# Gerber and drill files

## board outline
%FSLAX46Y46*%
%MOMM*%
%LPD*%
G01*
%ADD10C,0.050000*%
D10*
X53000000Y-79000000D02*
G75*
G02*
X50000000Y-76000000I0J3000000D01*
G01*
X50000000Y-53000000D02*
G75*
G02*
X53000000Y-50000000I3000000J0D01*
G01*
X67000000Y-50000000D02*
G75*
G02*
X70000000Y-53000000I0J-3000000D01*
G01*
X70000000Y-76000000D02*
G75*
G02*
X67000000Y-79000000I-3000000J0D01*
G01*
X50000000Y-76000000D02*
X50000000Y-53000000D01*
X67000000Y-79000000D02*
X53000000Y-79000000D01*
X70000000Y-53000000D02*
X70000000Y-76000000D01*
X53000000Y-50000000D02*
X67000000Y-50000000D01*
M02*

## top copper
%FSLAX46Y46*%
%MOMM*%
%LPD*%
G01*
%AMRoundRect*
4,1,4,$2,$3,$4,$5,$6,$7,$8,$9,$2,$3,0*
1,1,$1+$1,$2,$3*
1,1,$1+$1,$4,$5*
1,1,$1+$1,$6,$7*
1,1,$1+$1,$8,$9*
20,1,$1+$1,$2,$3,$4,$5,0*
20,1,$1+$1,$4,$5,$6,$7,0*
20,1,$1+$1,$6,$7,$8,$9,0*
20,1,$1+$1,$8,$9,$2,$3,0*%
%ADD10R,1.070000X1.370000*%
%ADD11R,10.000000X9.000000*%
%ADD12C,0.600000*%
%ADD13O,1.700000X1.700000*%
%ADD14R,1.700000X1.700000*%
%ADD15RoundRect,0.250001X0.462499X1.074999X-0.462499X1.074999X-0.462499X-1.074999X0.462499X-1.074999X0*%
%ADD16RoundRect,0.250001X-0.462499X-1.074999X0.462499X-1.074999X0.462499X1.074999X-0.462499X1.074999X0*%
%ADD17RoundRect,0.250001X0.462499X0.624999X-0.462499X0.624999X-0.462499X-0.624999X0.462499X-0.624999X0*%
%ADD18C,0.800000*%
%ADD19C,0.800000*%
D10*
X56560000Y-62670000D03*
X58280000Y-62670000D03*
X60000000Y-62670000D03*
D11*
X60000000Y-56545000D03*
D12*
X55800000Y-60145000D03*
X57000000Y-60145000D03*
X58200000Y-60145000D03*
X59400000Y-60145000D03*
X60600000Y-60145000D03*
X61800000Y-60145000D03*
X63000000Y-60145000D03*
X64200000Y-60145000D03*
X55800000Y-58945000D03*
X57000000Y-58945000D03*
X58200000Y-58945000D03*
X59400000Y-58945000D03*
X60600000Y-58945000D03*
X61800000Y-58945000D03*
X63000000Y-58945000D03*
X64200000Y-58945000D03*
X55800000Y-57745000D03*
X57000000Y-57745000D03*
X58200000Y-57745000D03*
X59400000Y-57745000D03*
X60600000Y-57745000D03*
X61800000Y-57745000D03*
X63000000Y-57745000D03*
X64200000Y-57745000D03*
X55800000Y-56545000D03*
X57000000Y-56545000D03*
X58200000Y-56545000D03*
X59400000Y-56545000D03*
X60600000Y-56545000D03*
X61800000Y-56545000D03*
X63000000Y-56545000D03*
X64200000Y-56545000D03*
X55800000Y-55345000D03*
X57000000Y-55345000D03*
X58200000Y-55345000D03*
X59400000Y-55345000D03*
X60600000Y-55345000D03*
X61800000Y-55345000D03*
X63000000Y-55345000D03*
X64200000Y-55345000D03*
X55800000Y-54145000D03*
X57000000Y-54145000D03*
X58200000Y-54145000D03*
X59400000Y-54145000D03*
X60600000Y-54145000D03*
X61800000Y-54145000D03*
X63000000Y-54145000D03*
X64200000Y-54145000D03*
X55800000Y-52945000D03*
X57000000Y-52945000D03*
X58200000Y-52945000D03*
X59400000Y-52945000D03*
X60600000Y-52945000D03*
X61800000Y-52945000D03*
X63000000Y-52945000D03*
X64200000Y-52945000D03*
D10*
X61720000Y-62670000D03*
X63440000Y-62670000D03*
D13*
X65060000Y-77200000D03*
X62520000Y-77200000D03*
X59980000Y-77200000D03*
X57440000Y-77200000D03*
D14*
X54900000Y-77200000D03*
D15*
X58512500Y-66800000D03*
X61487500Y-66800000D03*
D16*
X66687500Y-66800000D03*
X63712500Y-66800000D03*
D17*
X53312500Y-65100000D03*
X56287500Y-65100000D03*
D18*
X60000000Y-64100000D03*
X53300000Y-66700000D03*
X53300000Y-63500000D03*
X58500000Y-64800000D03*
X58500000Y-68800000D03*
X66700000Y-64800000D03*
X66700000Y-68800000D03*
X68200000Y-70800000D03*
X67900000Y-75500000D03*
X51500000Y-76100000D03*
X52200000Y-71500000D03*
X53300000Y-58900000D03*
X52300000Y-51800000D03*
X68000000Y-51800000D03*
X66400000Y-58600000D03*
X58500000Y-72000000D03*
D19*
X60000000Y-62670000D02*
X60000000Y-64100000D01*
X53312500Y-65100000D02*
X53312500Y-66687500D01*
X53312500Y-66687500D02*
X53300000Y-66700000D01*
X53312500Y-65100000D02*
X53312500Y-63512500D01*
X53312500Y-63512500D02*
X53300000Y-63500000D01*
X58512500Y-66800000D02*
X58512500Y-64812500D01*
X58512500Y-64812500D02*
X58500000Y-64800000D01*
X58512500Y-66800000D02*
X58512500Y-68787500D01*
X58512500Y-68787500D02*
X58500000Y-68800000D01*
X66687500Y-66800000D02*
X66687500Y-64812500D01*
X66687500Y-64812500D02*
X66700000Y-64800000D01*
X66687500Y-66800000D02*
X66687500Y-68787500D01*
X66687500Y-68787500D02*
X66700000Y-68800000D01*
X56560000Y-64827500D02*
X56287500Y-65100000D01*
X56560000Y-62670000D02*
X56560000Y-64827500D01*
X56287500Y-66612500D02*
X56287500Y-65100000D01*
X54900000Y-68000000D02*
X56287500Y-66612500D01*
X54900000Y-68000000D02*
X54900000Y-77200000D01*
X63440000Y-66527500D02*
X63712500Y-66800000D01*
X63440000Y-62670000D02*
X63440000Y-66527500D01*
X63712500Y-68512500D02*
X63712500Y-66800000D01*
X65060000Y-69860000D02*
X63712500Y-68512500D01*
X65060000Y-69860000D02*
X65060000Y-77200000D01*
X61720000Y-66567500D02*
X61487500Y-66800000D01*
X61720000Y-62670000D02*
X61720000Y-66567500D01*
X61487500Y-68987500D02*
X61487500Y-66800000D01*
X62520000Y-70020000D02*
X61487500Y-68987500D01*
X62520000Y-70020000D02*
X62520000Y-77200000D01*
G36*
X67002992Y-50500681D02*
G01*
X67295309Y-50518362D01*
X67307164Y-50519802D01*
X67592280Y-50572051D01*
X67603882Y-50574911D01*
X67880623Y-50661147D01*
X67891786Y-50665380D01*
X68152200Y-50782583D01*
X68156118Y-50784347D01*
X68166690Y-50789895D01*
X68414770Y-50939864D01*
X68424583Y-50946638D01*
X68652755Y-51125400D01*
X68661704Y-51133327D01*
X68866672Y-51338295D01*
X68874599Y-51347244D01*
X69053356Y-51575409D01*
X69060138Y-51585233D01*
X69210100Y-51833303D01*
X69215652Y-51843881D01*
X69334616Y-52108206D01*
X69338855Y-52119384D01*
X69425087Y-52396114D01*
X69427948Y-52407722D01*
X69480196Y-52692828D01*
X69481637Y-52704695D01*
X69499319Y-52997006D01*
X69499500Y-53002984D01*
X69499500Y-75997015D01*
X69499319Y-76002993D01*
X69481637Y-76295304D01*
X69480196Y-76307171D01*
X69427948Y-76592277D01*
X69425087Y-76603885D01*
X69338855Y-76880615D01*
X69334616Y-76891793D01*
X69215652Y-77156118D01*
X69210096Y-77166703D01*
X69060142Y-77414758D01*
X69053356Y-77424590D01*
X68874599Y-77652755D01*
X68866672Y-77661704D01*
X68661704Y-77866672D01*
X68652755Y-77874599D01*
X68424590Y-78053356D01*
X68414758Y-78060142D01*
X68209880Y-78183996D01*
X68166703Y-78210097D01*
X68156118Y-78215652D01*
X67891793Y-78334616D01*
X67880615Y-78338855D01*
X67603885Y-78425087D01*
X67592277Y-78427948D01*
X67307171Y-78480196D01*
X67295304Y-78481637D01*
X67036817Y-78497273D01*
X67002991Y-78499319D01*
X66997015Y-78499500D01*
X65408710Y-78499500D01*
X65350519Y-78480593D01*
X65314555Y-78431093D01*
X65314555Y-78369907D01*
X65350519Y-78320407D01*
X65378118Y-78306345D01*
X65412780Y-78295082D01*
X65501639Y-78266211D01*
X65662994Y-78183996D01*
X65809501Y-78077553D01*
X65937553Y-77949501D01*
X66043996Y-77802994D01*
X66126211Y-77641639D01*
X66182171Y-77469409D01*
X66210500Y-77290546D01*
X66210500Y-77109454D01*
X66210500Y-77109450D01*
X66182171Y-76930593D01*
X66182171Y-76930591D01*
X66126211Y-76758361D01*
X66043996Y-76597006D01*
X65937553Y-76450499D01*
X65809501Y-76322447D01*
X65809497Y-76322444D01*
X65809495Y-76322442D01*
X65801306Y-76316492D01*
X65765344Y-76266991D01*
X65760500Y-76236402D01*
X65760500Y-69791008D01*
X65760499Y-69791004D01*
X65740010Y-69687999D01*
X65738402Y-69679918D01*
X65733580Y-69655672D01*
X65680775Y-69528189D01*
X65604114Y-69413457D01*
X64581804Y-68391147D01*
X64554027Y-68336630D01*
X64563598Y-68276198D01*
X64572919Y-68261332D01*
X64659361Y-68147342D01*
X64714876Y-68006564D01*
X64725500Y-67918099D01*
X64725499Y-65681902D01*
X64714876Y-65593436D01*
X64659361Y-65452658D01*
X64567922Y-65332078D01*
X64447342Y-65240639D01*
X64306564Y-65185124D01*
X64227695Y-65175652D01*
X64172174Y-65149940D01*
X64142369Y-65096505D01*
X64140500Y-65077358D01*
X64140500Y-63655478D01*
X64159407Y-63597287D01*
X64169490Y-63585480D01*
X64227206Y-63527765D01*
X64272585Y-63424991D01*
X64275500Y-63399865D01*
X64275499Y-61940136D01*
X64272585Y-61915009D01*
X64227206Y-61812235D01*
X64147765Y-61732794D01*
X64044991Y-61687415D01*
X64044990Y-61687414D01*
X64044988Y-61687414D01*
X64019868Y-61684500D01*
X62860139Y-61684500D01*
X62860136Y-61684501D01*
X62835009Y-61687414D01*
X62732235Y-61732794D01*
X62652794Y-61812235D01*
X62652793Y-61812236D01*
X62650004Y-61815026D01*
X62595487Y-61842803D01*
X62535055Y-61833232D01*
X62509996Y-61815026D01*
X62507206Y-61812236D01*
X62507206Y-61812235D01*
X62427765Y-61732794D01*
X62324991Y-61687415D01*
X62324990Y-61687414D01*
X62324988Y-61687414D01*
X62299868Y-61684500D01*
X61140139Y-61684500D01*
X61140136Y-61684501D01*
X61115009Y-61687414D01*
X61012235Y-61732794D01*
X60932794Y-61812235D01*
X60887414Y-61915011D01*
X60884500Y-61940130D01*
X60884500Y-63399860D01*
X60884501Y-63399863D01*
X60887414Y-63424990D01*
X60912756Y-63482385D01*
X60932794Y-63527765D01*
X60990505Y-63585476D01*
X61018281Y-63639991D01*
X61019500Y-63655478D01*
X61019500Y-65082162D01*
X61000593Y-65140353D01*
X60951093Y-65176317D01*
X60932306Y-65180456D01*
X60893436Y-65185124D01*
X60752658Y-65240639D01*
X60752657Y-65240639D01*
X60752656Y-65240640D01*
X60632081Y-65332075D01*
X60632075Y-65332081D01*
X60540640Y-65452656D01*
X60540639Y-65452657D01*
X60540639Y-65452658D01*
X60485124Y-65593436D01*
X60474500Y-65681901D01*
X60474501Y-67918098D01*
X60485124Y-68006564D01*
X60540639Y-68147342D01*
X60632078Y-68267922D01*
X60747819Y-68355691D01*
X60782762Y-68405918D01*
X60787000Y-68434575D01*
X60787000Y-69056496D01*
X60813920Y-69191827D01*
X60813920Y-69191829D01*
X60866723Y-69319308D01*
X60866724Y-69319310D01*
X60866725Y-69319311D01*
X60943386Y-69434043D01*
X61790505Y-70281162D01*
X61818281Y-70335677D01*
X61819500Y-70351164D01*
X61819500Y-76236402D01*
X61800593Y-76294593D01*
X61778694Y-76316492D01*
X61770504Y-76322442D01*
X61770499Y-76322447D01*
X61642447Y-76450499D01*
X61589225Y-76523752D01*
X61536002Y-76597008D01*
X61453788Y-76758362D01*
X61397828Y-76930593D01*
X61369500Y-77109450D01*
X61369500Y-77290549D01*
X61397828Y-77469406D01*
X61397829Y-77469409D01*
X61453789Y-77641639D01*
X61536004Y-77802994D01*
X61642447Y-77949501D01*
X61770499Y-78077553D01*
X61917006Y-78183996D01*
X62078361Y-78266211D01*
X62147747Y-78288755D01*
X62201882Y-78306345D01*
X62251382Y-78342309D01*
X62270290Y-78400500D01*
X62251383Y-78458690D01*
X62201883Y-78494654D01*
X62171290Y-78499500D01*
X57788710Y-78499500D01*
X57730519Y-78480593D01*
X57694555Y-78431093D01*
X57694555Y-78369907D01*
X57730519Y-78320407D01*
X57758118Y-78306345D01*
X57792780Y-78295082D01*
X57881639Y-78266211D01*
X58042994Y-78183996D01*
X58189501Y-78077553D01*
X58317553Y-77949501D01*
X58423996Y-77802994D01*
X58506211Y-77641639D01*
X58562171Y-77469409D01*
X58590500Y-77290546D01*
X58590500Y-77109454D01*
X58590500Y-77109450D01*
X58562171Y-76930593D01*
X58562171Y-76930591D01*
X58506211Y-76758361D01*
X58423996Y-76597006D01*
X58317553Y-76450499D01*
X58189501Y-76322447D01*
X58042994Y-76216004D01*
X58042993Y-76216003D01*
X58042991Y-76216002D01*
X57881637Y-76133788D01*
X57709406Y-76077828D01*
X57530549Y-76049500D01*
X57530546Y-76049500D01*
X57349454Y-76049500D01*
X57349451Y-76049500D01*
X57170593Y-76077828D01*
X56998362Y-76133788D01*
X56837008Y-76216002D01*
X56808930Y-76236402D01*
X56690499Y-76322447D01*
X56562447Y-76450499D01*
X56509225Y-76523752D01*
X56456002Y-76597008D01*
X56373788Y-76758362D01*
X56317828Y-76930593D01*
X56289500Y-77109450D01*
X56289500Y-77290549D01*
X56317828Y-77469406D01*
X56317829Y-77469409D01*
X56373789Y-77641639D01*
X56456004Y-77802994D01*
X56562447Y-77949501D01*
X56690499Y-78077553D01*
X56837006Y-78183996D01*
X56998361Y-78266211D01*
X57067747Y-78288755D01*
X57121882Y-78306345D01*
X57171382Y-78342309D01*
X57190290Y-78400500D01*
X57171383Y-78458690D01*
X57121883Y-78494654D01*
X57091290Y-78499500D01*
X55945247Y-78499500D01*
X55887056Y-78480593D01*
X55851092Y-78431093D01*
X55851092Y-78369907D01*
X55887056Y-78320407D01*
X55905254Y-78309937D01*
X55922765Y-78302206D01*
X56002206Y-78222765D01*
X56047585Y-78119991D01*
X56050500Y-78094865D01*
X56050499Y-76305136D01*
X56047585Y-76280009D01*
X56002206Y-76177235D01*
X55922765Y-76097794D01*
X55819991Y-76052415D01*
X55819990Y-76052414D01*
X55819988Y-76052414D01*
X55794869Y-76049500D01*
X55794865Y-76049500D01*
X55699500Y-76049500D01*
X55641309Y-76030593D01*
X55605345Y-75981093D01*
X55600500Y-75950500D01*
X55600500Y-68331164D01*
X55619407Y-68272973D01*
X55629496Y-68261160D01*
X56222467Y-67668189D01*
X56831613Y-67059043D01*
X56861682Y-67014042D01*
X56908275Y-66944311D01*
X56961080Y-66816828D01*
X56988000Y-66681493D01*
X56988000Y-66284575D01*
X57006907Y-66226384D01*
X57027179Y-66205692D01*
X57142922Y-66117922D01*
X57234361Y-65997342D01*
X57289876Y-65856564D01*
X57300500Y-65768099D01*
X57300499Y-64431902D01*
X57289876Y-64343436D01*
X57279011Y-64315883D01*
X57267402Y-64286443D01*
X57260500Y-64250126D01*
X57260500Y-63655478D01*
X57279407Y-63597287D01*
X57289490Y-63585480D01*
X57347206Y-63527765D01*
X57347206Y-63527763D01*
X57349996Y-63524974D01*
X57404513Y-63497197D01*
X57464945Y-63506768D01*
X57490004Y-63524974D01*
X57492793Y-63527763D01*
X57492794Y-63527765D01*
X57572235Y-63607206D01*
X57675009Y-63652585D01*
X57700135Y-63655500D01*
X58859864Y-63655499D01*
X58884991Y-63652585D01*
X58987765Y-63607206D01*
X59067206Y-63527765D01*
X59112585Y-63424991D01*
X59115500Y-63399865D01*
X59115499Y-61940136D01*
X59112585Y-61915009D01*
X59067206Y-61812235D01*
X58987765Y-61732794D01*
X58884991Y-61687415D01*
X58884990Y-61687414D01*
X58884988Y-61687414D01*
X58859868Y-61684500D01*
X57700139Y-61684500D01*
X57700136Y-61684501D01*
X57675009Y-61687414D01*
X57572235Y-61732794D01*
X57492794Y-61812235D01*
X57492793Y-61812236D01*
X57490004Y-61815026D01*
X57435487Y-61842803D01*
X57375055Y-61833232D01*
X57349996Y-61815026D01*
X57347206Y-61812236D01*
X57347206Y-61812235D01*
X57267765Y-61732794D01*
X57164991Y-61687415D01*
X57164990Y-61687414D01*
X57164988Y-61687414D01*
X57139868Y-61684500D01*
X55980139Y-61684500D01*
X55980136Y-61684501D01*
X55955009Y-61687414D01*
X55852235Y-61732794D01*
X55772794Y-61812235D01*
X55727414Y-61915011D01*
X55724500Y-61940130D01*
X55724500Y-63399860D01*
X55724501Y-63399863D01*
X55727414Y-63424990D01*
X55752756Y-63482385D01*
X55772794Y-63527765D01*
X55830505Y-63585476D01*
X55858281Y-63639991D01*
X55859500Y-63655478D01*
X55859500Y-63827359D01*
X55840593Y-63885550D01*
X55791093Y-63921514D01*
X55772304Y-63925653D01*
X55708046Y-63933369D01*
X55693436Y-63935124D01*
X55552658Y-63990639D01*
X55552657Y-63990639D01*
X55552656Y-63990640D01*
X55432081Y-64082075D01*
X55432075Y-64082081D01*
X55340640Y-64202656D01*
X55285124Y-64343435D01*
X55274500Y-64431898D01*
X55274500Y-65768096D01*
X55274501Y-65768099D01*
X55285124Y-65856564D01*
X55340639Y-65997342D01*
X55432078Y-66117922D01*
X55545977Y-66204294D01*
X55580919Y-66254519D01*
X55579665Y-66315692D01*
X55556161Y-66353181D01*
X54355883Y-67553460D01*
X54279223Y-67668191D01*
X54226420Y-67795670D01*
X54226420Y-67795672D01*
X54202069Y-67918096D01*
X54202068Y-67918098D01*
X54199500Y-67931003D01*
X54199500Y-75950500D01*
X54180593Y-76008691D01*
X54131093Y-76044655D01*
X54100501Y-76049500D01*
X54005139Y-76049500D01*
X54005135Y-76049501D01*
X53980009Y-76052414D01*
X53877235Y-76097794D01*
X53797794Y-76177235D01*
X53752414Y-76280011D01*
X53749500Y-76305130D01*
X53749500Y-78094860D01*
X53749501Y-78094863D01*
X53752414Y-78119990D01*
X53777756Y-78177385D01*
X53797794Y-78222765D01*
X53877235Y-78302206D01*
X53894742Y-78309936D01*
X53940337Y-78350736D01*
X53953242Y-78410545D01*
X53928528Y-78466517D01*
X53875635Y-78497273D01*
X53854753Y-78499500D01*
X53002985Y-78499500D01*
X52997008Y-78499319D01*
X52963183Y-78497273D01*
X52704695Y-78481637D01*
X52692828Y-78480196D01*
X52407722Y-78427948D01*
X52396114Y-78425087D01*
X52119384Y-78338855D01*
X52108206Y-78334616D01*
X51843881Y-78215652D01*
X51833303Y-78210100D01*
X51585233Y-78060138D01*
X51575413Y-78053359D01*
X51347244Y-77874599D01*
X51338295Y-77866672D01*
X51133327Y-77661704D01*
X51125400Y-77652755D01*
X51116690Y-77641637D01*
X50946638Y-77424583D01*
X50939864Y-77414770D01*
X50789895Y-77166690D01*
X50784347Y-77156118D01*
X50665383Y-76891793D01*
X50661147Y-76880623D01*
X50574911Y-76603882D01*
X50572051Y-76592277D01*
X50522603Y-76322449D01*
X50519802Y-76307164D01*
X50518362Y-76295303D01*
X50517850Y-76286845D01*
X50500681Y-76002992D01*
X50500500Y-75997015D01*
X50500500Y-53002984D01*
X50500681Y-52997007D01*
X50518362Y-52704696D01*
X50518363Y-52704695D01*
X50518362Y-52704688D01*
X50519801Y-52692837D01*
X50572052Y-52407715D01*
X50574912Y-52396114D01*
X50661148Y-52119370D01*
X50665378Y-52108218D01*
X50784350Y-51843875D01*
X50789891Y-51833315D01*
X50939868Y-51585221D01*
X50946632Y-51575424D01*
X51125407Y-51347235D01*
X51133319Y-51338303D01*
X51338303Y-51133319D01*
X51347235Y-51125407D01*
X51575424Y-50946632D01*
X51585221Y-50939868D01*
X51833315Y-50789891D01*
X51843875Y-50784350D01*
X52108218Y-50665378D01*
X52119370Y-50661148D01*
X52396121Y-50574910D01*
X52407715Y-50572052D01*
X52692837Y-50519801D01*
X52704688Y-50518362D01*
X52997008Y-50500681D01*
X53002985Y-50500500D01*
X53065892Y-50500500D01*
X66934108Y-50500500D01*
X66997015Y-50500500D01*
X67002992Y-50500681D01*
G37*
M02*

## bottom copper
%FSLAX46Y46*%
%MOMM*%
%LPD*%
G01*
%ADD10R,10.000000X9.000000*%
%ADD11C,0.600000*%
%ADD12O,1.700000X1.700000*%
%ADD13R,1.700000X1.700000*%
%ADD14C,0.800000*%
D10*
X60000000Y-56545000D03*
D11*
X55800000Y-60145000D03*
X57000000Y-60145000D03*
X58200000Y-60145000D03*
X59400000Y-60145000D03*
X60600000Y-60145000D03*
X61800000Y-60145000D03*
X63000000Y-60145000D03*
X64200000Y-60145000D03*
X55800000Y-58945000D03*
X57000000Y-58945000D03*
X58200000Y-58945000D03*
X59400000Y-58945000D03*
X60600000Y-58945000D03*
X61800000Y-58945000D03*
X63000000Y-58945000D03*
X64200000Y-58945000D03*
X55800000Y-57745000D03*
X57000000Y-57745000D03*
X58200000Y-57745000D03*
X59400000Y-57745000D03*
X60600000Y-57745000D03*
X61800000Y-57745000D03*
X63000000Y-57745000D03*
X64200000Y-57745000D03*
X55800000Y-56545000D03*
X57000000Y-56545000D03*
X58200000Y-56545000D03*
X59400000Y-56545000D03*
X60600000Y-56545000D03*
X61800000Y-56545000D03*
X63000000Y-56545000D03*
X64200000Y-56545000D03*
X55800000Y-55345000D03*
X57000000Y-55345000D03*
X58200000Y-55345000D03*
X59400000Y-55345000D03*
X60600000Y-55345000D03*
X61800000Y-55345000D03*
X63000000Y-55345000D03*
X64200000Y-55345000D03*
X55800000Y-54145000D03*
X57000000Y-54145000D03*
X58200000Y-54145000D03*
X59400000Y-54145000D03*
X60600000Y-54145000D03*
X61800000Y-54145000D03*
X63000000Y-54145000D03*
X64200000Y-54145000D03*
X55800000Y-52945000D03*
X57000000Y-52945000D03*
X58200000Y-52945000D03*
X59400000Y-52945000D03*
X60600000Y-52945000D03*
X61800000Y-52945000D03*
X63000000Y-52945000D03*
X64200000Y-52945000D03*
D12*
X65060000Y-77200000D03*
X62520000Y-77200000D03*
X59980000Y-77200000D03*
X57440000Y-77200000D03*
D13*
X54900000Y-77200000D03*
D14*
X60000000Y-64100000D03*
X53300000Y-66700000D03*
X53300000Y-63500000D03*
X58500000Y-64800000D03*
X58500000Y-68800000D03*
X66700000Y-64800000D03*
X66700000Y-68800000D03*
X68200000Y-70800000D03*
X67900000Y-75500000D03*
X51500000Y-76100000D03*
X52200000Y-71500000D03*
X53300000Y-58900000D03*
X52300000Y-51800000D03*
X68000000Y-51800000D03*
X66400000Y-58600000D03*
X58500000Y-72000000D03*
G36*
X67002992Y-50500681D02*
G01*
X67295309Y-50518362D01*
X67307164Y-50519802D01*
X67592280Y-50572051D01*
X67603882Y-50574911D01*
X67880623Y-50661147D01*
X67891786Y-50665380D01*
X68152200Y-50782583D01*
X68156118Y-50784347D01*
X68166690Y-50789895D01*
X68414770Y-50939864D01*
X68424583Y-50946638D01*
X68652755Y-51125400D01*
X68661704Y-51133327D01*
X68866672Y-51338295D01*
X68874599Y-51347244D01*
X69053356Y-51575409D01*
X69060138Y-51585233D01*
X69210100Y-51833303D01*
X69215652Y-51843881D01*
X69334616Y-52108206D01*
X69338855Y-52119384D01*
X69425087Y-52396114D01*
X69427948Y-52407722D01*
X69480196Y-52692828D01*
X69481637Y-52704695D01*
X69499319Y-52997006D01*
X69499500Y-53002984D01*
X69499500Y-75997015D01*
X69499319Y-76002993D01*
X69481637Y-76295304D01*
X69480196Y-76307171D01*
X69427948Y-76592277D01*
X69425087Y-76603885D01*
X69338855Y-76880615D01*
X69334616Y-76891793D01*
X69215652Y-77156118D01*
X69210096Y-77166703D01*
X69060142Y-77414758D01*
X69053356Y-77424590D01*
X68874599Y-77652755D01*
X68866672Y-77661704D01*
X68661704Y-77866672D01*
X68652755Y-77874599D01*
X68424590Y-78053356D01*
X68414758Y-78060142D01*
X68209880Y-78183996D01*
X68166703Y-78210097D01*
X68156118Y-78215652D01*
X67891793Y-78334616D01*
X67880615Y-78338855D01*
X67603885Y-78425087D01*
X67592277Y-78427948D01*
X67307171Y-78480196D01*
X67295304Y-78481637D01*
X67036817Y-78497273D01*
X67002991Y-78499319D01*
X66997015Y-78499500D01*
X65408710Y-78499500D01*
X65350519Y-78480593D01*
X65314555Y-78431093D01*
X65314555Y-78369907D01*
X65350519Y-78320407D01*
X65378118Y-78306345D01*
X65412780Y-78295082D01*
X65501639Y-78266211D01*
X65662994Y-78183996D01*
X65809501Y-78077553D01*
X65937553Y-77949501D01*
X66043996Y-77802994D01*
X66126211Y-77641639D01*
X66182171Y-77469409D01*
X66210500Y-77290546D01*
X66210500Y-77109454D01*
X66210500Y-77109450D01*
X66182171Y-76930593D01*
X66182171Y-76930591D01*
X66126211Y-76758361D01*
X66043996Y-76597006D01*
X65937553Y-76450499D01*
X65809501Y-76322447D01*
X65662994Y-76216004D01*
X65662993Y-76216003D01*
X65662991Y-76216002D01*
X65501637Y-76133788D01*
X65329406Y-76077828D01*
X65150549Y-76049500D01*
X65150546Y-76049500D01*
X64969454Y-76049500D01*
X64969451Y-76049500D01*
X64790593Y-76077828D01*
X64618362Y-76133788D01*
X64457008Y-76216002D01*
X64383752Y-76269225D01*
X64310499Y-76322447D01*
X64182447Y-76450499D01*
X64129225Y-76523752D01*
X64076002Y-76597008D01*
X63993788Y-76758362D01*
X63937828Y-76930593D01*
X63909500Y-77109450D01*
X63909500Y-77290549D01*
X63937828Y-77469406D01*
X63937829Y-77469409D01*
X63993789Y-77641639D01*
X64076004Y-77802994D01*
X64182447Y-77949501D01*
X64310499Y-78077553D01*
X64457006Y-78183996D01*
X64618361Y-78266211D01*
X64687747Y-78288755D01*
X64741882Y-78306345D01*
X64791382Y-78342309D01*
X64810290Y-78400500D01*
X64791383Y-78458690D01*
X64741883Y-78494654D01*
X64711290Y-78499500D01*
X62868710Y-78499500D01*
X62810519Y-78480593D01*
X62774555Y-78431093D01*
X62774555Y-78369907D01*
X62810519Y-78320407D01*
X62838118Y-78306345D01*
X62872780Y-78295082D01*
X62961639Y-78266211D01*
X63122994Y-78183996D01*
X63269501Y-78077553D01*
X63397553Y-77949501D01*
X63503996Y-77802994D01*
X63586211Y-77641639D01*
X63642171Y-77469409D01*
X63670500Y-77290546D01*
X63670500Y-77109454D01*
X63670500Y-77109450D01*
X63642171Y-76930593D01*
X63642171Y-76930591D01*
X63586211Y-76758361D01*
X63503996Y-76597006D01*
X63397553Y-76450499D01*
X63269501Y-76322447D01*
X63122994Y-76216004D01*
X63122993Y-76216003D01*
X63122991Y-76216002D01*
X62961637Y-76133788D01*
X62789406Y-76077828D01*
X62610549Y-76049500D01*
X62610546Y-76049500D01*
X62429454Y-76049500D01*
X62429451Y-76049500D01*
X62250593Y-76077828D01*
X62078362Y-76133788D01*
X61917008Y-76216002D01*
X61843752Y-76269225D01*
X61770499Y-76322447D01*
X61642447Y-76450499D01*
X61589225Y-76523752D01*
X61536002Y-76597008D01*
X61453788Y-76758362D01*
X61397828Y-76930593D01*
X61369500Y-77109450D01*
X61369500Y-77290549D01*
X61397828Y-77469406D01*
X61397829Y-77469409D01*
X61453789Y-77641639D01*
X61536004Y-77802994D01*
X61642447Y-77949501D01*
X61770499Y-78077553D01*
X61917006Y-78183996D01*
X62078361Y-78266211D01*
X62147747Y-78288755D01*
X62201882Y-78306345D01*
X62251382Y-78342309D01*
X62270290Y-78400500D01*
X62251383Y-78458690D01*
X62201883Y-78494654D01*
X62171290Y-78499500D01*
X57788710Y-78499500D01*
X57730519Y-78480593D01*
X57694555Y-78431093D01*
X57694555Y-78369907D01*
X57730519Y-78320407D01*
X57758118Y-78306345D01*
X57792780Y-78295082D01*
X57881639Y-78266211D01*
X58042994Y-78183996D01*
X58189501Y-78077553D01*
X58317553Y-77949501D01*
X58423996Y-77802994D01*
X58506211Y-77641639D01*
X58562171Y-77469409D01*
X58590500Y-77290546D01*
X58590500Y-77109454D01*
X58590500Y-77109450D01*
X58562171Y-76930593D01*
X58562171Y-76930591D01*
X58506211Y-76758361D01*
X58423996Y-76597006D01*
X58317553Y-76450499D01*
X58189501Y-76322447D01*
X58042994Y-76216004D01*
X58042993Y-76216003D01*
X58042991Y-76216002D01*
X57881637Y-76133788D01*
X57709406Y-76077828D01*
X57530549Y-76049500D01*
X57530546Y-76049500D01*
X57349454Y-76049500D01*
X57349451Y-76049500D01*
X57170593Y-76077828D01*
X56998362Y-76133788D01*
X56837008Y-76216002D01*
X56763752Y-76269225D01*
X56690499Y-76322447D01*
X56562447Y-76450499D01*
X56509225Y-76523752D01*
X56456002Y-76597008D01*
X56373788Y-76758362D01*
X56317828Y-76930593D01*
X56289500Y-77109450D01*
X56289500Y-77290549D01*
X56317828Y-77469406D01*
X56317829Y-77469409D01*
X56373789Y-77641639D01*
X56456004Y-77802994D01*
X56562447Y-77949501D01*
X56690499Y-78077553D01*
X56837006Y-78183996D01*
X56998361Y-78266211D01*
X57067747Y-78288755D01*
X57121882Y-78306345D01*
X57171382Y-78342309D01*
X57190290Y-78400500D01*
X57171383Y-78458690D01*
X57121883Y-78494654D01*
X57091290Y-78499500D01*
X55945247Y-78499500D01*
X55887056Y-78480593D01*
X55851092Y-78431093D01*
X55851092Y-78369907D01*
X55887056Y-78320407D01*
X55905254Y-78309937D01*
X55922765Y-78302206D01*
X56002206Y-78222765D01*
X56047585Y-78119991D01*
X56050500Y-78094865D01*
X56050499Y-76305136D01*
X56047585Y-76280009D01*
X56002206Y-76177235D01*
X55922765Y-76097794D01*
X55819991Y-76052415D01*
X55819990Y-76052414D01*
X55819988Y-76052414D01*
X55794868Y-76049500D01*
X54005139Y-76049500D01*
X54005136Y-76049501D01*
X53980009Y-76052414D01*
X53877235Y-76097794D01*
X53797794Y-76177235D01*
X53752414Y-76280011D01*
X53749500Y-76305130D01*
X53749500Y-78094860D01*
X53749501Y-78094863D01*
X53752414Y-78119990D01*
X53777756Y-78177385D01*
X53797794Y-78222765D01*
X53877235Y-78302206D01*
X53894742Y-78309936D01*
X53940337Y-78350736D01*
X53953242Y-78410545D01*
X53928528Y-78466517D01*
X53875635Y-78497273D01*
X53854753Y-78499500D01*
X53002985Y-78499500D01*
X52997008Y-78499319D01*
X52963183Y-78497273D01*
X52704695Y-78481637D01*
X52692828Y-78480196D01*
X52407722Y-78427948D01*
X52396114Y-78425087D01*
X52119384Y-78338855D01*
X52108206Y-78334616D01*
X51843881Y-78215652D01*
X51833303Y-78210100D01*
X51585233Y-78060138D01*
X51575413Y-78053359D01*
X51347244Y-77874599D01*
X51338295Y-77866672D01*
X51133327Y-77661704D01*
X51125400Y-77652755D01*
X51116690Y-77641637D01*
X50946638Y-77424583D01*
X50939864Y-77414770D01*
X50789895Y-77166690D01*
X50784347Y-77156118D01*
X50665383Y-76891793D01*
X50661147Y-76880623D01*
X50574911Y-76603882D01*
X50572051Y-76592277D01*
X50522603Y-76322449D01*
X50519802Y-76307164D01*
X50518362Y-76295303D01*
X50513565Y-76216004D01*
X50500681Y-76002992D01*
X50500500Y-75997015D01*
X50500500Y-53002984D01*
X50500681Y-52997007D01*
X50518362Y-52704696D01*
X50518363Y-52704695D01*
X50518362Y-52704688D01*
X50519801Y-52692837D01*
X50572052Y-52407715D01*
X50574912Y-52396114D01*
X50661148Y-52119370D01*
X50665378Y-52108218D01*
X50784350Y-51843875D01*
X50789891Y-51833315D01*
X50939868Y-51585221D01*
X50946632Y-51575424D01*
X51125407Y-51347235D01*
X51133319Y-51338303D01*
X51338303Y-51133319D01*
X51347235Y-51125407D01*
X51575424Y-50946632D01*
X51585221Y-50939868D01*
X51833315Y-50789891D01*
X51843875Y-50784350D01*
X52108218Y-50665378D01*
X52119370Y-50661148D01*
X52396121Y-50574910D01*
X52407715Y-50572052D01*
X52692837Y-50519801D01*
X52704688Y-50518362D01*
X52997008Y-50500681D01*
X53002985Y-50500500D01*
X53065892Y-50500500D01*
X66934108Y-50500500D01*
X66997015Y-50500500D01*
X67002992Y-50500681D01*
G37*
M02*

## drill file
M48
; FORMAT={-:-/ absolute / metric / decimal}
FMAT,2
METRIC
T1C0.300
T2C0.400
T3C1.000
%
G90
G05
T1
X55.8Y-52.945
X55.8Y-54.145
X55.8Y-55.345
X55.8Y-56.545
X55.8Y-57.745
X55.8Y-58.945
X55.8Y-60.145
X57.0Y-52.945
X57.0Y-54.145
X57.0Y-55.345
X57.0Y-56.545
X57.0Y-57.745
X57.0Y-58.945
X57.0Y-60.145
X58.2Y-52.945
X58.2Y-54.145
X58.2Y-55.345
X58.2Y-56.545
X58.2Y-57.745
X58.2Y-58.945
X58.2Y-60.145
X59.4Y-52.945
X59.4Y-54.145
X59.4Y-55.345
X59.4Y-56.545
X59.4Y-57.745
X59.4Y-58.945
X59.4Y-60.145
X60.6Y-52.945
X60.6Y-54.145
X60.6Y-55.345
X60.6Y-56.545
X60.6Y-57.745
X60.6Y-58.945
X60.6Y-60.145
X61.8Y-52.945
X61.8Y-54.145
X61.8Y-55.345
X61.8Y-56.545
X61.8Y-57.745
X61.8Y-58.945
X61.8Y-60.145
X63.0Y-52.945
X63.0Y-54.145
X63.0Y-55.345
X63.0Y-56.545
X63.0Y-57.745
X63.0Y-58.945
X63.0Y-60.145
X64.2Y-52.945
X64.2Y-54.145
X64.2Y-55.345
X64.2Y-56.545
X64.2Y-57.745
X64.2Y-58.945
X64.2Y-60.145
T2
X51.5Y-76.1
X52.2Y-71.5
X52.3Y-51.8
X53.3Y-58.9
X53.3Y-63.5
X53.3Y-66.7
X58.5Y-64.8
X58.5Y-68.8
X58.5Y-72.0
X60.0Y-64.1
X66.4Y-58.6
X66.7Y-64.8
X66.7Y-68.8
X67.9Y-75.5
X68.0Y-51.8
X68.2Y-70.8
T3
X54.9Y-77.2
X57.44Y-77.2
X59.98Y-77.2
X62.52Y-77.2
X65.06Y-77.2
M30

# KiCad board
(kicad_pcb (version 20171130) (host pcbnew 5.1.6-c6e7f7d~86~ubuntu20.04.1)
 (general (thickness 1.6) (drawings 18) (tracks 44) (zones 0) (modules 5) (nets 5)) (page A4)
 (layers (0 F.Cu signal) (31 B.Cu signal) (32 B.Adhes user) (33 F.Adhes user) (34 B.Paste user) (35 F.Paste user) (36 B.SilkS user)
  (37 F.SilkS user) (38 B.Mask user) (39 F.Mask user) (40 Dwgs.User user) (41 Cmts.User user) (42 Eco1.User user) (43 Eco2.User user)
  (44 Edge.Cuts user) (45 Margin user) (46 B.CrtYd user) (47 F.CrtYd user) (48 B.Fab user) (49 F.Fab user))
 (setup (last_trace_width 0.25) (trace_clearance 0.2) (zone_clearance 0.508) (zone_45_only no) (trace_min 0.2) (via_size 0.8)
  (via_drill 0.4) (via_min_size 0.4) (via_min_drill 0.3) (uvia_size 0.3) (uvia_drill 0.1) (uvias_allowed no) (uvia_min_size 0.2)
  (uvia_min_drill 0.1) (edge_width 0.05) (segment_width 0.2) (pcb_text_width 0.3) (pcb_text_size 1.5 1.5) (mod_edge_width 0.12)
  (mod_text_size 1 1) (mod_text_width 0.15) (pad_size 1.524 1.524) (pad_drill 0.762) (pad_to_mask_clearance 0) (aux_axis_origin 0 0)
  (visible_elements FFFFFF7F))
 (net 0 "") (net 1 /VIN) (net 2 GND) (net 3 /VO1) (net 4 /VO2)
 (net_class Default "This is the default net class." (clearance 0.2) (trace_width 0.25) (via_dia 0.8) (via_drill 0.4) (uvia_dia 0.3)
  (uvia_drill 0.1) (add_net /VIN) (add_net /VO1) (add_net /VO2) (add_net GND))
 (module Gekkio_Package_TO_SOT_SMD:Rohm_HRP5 (layer F.Cu) (at 60 57.7 90)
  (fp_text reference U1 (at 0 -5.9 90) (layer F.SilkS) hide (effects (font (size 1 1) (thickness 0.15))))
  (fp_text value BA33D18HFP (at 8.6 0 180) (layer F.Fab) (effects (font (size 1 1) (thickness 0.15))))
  (pad 1 smd rect (at -4.97 -3.44 90) (size 1.37 1.07) (layers F.Cu F.Paste F.Mask) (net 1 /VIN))
  (pad 2 smd rect (at -4.97 -1.72 90) (size 1.37 1.07) (layers F.Cu F.Paste F.Mask))
  (pad 3 smd rect (at -4.97 0 90) (size 1.37 1.07) (layers F.Cu F.Paste F.Mask) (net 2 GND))
  (pad 3 smd rect (at 1.155 0 90) (size 9 10) (layers F.Cu F.Mask) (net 2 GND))
  (pad 3 smd rect (at 1.155 0 90) (size 9 10) (layers B.Cu) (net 2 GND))
  (pad "" smd rect (at -1.095 2.5 90) (size 4 4.5) (layers F.Paste))
  (pad "" smd rect (at 3.405 -2.5 90) (size 4 4.5) (layers F.Paste))
  (pad "" smd rect (at -1.095 -2.5 90) (size 4 4.5) (layers F.Paste))
  (pad "" smd rect (at 3.405 2.5 90) (size 4 4.5) (layers F.Paste))
  (pad 3 thru_hole circle (at -2.445 -4.2 90) (size 0.6 0.6) (drill 0.3) (layers *.Cu) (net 2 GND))
  (pad 3 thru_hole circle (at -2.445 -3 90) (size 0.6 0.6) (drill 0.3) (layers *.Cu) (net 2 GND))
  (pad 3 thru_hole circle (at -2.445 -1.8 90) (size 0.6 0.6) (drill 0.3) (layers *.Cu) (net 2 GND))
  (pad 3 thru_hole circle (at -2.445 -0.6 90) (size 0.6 0.6) (drill 0.3) (layers *.Cu) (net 2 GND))
  (pad 3 thru_hole circle (at -2.445 0.6 90) (size 0.6 0.6) (drill 0.3) (layers *.Cu) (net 2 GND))
  (pad 3 thru_hole circle (at -2.445 1.8 90) (size 0.6 0.6) (drill 0.3) (layers *.Cu) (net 2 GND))
  (pad 3 thru_hole circle (at -2.445 3 90) (size 0.6 0.6) (drill 0.3) (layers *.Cu) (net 2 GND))
  (pad 3 thru_hole circle (at -2.445 4.2 90) (size 0.6 0.6) (drill 0.3) (layers *.Cu) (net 2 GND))
  (pad 3 thru_hole circle (at -1.245 -4.2 90) (size 0.6 0.6) (drill 0.3) (layers *.Cu) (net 2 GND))
  (pad 3 thru_hole circle (at -1.245 -3 90) (size 0.6 0.6) (drill 0.3) (layers *.Cu) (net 2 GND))
  (pad 3 thru_hole circle (at -1.245 -1.8 90) (size 0.6 0.6) (drill 0.3) (layers *.Cu) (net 2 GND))
  (pad 3 thru_hole circle (at -1.245 -0.6 90) (size 0.6 0.6) (drill 0.3) (layers *.Cu) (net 2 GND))
  (pad 3 thru_hole circle (at -1.245 0.6 90) (size 0.6 0.6) (drill 0.3) (layers *.Cu) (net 2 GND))
  (pad 3 thru_hole circle (at -1.245 1.8 90) (size 0.6 0.6) (drill 0.3) (layers *.Cu) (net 2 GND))
  (pad 3 thru_hole circle (at -1.245 3 90) (size 0.6 0.6) (drill 0.3) (layers *.Cu) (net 2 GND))
  (pad 3 thru_hole circle (at -1.245 4.2 90) (size 0.6 0.6) (drill 0.3) (layers *.Cu) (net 2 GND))
  (pad 3 thru_hole circle (at -0.045 -4.2 90) (size 0.6 0.6) (drill 0.3) (layers *.Cu) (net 2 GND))
  (pad 3 thru_hole circle (at -0.045 -3 90) (size 0.6 0.6) (drill 0.3) (layers *.Cu) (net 2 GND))
  (pad 3 thru_hole circle (at -0.045 -1.8 90) (size 0.6 0.6) (drill 0.3) (layers *.Cu) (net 2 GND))
  (pad 3 thru_hole circle (at -0.045 -0.6 90) (size 0.6 0.6) (drill 0.3) (layers *.Cu) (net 2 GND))
  (pad 3 thru_hole circle (at -0.045 0.6 90) (size 0.6 0.6) (drill 0.3) (layers *.Cu) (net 2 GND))
  (pad 3 thru_hole circle (at -0.045 1.8 90) (size 0.6 0.6) (drill 0.3) (layers *.Cu) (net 2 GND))
  (pad 3 thru_hole circle (at -0.045 3 90) (size 0.6 0.6) (drill 0.3) (layers *.Cu) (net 2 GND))
  (pad 3 thru_hole circle (at -0.045 4.2 90) (size 0.6 0.6) (drill 0.3) (layers *.Cu) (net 2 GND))
  (pad 3 thru_hole circle (at 1.155 -4.2 90) (size 0.6 0.6) (drill 0.3) (layers *.Cu) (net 2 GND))
  (pad 3 thru_hole circle (at 1.155 -3 90) (size 0.6 0.6) (drill 0.3) (layers *.Cu) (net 2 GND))
  (pad 3 thru_hole circle (at 1.155 -1.8 90) (size 0.6 0.6) (drill 0.3) (layers *.Cu) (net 2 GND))
  (pad 3 thru_hole circle (at 1.155 -0.6 90) (size 0.6 0.6) (drill 0.3) (layers *.Cu) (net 2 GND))
  (pad 3 thru_hole circle (at 1.155 0.6 90) (size 0.6 0.6) (drill 0.3) (layers *.Cu) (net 2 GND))
  (pad 3 thru_hole circle (at 1.155 1.8 90) (size 0.6 0.6) (drill 0.3) (layers *.Cu) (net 2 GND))
  (pad 3 thru_hole circle (at 1.155 3 90) (size 0.6 0.6) (drill 0.3) (layers *.Cu) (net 2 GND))
  (pad 3 thru_hole circle (at 1.155 4.2 90) (size 0.6 0.6) (drill 0.3) (layers *.Cu) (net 2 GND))
  (pad 3 thru_hole circle (at 2.355 -4.2 90) (size 0.6 0.6) (drill 0.3) (layers *.Cu) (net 2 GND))
  (pad 3 thru_hole circle (at 2.355 -3 90) (size 0.6 0.6) (drill 0.3) (layers *.Cu) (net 2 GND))
  (pad 3 thru_hole circle (at 2.355 -1.8 90) (size 0.6 0.6) (drill 0.3) (layers *.Cu) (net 2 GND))
  (pad 3 thru_hole circle (at 2.355 -0.6 90) (size 0.6 0.6) (drill 0.3) (layers *.Cu) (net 2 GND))
  (pad 3 thru_hole circle (at 2.355 0.6 90) (size 0.6 0.6) (drill 0.3) (layers *.Cu) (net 2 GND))
  (pad 3 thru_hole circle (at 2.355 1.8 90) (size 0.6 0.6) (drill 0.3) (layers *.Cu) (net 2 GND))
  (pad 3 thru_hole circle (at 2.355 3 90) (size 0.6 0.6) (drill 0.3) (layers *.Cu) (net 2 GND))
  (pad 3 thru_hole circle (at 2.355 4.2 90) (size 0.6 0.6) (drill 0.3) (layers *.Cu) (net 2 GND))
  (pad 3 thru_hole circle (at 3.555 -4.2 90) (size 0.6 0.6) (drill 0.3) (layers *.Cu) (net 2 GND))
  (pad 3 thru_hole circle (at 3.555 -3 90) (size 0.6 0.6) (drill 0.3) (layers *.Cu) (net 2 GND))
  (pad 3 thru_hole circle (at 3.555 -1.8 90) (size 0.6 0.6) (drill 0.3) (layers *.Cu) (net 2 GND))
  (pad 3 thru_hole circle (at 3.555 -0.6 90) (size 0.6 0.6) (drill 0.3) (layers *.Cu) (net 2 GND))
  (pad 3 thru_hole circle (at 3.555 0.6 90) (size 0.6 0.6) (drill 0.3) (layers *.Cu) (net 2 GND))
  (pad 3 thru_hole circle (at 3.555 1.8 90) (size 0.6 0.6) (drill 0.3) (layers *.Cu) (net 2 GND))
  (pad 3 thru_hole circle (at 3.555 3 90) (size 0.6 0.6) (drill 0.3) (layers *.Cu) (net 2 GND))
  (pad 3 thru_hole circle (at 3.555 4.2 90) (size 0.6 0.6) (drill 0.3) (layers *.Cu) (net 2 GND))
  (pad 3 thru_hole circle (at 4.755 -4.2 90) (size 0.6 0.6) (drill 0.3) (layers *.Cu) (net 2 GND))
  (pad 3 thru_hole circle (at 4.755 -3 90) (size 0.6 0.6) (drill 0.3) (layers *.Cu) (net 2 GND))
  (pad 3 thru_hole circle (at 4.755 -1.8 90) (size 0.6 0.6) (drill 0.3) (layers *.Cu) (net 2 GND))
  (pad 3 thru_hole circle (at 4.755 -0.6 90) (size 0.6 0.6) (drill 0.3) (layers *.Cu) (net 2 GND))
  (pad 3 thru_hole circle (at 4.755 0.6 90) (size 0.6 0.6) (drill 0.3) (layers *.Cu) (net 2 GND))
  (pad 3 thru_hole circle (at 4.755 1.8 90) (size 0.6 0.6) (drill 0.3) (layers *.Cu) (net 2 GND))
  (pad 3 thru_hole circle (at 4.755 3 90) (size 0.6 0.6) (drill 0.3) (layers *.Cu) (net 2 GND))
  (pad 3 thru_hole circle (at 4.755 4.2 90) (size 0.6 0.6) (drill 0.3) (layers *.Cu) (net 2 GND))
  (pad 4 smd rect (at -4.97 1.72 90) (size 1.37 1.07) (layers F.Cu F.Paste F.Mask) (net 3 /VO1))
  (pad 5 smd rect (at -4.97 3.44 90) (size 1.37 1.07) (layers F.Cu F.Paste F.Mask) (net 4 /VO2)))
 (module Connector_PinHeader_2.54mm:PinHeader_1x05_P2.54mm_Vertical (layer F.Cu) (at 54.9 77.2 90)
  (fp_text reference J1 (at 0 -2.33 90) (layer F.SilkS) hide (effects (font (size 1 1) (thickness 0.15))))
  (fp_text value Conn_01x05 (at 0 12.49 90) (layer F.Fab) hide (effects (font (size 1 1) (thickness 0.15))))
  (pad 5 thru_hole oval (at 0 10.16 90) (size 1.7 1.7) (drill 1) (layers *.Cu *.Mask) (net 4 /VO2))
  (pad 4 thru_hole oval (at 0 7.62 90) (size 1.7 1.7) (drill 1) (layers *.Cu *.Mask) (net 3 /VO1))
  (pad 3 thru_hole oval (at 0 5.08 90) (size 1.7 1.7) (drill 1) (layers *.Cu *.Mask) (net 2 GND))
  (pad 2 thru_hole oval (at 0 2.54 90) (size 1.7 1.7) (drill 1) (layers *.Cu *.Mask))
  (pad 1 thru_hole rect (at 0 0 90) (size 1.7 1.7) (drill 1) (layers *.Cu *.Mask) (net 1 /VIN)))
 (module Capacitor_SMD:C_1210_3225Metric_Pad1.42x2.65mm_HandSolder (layer F.Cu) (at 60 66.8 180)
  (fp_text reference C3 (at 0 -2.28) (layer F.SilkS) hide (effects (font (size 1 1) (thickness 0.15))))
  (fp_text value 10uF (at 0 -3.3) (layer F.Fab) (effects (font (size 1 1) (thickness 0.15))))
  (pad 2 smd roundrect (at 1.4875 0 180) (size 1.425 2.65) (layers F.Cu F.Paste F.Mask) (roundrect_rratio 0.175439) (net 2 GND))
  (pad 1 smd roundrect (at -1.4875 0 180) (size 1.425 2.65) (layers F.Cu F.Paste F.Mask) (roundrect_rratio 0.175439) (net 3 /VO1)))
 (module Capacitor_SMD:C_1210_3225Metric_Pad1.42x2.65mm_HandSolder (layer F.Cu) (at 65.2 66.8)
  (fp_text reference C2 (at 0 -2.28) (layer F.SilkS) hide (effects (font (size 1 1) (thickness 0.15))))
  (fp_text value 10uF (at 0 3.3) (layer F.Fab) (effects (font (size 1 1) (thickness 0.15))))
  (pad 2 smd roundrect (at 1.4875 0) (size 1.425 2.65) (layers F.Cu F.Paste F.Mask) (roundrect_rratio 0.175439) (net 2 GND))
  (pad 1 smd roundrect (at -1.4875 0) (size 1.425 2.65) (layers F.Cu F.Paste F.Mask) (roundrect_rratio 0.175439) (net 4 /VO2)))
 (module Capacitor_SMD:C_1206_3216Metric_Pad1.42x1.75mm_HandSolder (layer F.Cu) (at 54.8 65.1 180)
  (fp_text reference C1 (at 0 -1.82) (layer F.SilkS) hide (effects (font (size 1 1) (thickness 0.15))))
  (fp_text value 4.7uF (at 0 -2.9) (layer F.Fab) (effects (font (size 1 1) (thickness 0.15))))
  (pad 2 smd roundrect (at 1.4875 0 180) (size 1.425 1.75) (layers F.Cu F.Paste F.Mask) (roundrect_rratio 0.175439) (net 2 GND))
  (pad 1 smd roundrect (at -1.4875 0 180) (size 1.425 1.75) (layers F.Cu F.Paste F.Mask) (roundrect_rratio 0.175439) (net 1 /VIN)))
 (gr_arc (start 53 76) (end 50 76) (angle -90) (layer Edge.Cuts) (width 0.05))
 (gr_arc (start 53 53) (end 53 50) (angle -90) (layer Edge.Cuts) (width 0.05))
 (gr_arc (start 67 53) (end 70 53) (angle -90) (layer Edge.Cuts) (width 0.05))
 (gr_arc (start 67 76) (end 67 79) (angle -90) (layer Edge.Cuts) (width 0.05))
 (gr_line (start 50 76) (end 50 53) (layer Edge.Cuts) (width 0.05))
 (gr_line (start 67 79) (end 53 79) (layer Edge.Cuts) (width 0.05))
 (gr_line (start 70 53) (end 70 76) (layer Edge.Cuts) (width 0.05))
 (gr_line (start 53 50) (end 67 50) (layer Edge.Cuts) (width 0.05))
 (via (at 60 64.1) (size 0.8) (drill 0.4) (layers F.Cu B.Cu) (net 2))
 (segment (start 60 62.67) (end 60 64.1) (width 0.8) (layer F.Cu) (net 2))
 (via (at 53.3 66.7) (size 0.8) (drill 0.4) (layers F.Cu B.Cu) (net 2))
 (segment (start 53.3125 65.1) (end 53.3125 66.6875) (width 0.8) (layer F.Cu) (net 2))
 (segment (start 53.3125 66.6875) (end 53.3 66.7) (width 0.8) (layer F.Cu) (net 2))
 (via (at 53.3 63.5) (size 0.8) (drill 0.4) (layers F.Cu B.Cu) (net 2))
 (segment (start 53.3125 65.1) (end 53.3125 63.5125) (width 0.8) (layer F.Cu) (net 2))
 (segment (start 53.3125 63.5125) (end 53.3 63.5) (width 0.8) (layer F.Cu) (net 2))
 (via (at 58.5 64.8) (size 0.8) (drill 0.4) (layers F.Cu B.Cu) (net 2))
 (segment (start 58.5125 66.8) (end 58.5125 64.8125) (width 0.8) (layer F.Cu) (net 2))
 (segment (start 58.5125 64.8125) (end 58.5 64.8) (width 0.8) (layer F.Cu) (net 2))
 (via (at 58.5 68.8) (size 0.8) (drill 0.4) (layers F.Cu B.Cu) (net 2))
 (segment (start 58.5125 66.8) (end 58.5125 68.7875) (width 0.8) (layer F.Cu) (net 2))
 (segment (start 58.5125 68.7875) (end 58.5 68.8) (width 0.8) (layer F.Cu) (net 2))
 (via (at 66.7 64.8) (size 0.8) (drill 0.4) (layers F.Cu B.Cu) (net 2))
 (segment (start 66.6875 66.8) (end 66.6875 64.8125) (width 0.8) (layer F.Cu) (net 2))
 (segment (start 66.6875 64.8125) (end 66.7 64.8) (width 0.8) (layer F.Cu) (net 2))
 (segment (start 66.6875 66.8) (end 66.6875 68.7875) (width 0.8) (layer F.Cu) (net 2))
 (via (at 66.7 68.8) (size 0.8) (drill 0.4) (layers F.Cu B.Cu) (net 2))
 (segment (start 66.6875 68.7875) (end 66.7 68.8) (width 0.8) (layer F.Cu) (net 2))
 (via (at 68.2 70.8) (size 0.8) (drill 0.4) (layers F.Cu B.Cu) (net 2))
 (via (at 67.9 75.5) (size 0.8) (drill 0.4) (layers F.Cu B.Cu) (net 2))
 (via (at 51.5 76.1) (size 0.8) (drill 0.4) (layers F.Cu B.Cu) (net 2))
 (via (at 52.2 71.5) (size 0.8) (drill 0.4) (layers F.Cu B.Cu) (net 2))
 (via (at 53.3 58.9) (size 0.8) (drill 0.4) (layers F.Cu B.Cu) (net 2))
 (via (at 52.3 51.8) (size 0.8) (drill 0.4) (layers F.Cu B.Cu) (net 2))
 (via (at 68 51.8) (size 0.8) (drill 0.4) (layers F.Cu B.Cu) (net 2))
 (via (at 66.4 58.6) (size 0.8) (drill 0.4) (layers F.Cu B.Cu) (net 2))
 (via (at 58.5 72) (size 0.8) (drill 0.4) (layers F.Cu B.Cu) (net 2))
 (segment (start 56.56 64.8275) (end 56.2875 65.1) (width 0.8) (layer F.Cu) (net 1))
 (segment (start 56.56 62.67) (end 56.56 64.8275) (width 0.8) (layer F.Cu) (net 1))
 (segment (start 56.2875 66.6125) (end 56.2875 65.1) (width 0.8) (layer F.Cu) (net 1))
 (segment (start 54.9 68) (end 56.2875 66.6125) (width 0.8) (layer F.Cu) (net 1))
 (segment (start 54.9 68) (end 54.9 77.2) (width 0.8) (layer F.Cu) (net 1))
 (segment (start 63.44 66.5275) (end 63.7125 66.8) (width 0.8) (layer F.Cu) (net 4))
 (segment (start 63.44 62.67) (end 63.44 66.5275) (width 0.8) (layer F.Cu) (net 4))
 (segment (start 63.7125 68.5125) (end 63.7125 66.8) (width 0.8) (layer F.Cu) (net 4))
 (segment (start 65.06 69.86) (end 63.7125 68.5125) (width 0.8) (layer F.Cu) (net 4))
 (segment (start 65.06 69.86) (end 65.06 77.2) (width 0.8) (layer F.Cu) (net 4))
 (segment (start 61.72 66.5675) (end 61.4875 66.8) (width 0.8) (layer F.Cu) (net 3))
 (segment (start 61.72 62.67) (end 61.72 66.5675) (width 0.8) (layer F.Cu) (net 3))
 (segment (start 61.4875 68.9875) (end 61.4875 66.8) (width 0.8) (layer F.Cu) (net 3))
 (segment (start 62.52 70.02) (end 61.4875 68.9875) (width 0.8) (layer F.Cu) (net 3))
 (segment (start 62.52 70.02) (end 62.52 77.2) (width 0.8) (layer F.Cu) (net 3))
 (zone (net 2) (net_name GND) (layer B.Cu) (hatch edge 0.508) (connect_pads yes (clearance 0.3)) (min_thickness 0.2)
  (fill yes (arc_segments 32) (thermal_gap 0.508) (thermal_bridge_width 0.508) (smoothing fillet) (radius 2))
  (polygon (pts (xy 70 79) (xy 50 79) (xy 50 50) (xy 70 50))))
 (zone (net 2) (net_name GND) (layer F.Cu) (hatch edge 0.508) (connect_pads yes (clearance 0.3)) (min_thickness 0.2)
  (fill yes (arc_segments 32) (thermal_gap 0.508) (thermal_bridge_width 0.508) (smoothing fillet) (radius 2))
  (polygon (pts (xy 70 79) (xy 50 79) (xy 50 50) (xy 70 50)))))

